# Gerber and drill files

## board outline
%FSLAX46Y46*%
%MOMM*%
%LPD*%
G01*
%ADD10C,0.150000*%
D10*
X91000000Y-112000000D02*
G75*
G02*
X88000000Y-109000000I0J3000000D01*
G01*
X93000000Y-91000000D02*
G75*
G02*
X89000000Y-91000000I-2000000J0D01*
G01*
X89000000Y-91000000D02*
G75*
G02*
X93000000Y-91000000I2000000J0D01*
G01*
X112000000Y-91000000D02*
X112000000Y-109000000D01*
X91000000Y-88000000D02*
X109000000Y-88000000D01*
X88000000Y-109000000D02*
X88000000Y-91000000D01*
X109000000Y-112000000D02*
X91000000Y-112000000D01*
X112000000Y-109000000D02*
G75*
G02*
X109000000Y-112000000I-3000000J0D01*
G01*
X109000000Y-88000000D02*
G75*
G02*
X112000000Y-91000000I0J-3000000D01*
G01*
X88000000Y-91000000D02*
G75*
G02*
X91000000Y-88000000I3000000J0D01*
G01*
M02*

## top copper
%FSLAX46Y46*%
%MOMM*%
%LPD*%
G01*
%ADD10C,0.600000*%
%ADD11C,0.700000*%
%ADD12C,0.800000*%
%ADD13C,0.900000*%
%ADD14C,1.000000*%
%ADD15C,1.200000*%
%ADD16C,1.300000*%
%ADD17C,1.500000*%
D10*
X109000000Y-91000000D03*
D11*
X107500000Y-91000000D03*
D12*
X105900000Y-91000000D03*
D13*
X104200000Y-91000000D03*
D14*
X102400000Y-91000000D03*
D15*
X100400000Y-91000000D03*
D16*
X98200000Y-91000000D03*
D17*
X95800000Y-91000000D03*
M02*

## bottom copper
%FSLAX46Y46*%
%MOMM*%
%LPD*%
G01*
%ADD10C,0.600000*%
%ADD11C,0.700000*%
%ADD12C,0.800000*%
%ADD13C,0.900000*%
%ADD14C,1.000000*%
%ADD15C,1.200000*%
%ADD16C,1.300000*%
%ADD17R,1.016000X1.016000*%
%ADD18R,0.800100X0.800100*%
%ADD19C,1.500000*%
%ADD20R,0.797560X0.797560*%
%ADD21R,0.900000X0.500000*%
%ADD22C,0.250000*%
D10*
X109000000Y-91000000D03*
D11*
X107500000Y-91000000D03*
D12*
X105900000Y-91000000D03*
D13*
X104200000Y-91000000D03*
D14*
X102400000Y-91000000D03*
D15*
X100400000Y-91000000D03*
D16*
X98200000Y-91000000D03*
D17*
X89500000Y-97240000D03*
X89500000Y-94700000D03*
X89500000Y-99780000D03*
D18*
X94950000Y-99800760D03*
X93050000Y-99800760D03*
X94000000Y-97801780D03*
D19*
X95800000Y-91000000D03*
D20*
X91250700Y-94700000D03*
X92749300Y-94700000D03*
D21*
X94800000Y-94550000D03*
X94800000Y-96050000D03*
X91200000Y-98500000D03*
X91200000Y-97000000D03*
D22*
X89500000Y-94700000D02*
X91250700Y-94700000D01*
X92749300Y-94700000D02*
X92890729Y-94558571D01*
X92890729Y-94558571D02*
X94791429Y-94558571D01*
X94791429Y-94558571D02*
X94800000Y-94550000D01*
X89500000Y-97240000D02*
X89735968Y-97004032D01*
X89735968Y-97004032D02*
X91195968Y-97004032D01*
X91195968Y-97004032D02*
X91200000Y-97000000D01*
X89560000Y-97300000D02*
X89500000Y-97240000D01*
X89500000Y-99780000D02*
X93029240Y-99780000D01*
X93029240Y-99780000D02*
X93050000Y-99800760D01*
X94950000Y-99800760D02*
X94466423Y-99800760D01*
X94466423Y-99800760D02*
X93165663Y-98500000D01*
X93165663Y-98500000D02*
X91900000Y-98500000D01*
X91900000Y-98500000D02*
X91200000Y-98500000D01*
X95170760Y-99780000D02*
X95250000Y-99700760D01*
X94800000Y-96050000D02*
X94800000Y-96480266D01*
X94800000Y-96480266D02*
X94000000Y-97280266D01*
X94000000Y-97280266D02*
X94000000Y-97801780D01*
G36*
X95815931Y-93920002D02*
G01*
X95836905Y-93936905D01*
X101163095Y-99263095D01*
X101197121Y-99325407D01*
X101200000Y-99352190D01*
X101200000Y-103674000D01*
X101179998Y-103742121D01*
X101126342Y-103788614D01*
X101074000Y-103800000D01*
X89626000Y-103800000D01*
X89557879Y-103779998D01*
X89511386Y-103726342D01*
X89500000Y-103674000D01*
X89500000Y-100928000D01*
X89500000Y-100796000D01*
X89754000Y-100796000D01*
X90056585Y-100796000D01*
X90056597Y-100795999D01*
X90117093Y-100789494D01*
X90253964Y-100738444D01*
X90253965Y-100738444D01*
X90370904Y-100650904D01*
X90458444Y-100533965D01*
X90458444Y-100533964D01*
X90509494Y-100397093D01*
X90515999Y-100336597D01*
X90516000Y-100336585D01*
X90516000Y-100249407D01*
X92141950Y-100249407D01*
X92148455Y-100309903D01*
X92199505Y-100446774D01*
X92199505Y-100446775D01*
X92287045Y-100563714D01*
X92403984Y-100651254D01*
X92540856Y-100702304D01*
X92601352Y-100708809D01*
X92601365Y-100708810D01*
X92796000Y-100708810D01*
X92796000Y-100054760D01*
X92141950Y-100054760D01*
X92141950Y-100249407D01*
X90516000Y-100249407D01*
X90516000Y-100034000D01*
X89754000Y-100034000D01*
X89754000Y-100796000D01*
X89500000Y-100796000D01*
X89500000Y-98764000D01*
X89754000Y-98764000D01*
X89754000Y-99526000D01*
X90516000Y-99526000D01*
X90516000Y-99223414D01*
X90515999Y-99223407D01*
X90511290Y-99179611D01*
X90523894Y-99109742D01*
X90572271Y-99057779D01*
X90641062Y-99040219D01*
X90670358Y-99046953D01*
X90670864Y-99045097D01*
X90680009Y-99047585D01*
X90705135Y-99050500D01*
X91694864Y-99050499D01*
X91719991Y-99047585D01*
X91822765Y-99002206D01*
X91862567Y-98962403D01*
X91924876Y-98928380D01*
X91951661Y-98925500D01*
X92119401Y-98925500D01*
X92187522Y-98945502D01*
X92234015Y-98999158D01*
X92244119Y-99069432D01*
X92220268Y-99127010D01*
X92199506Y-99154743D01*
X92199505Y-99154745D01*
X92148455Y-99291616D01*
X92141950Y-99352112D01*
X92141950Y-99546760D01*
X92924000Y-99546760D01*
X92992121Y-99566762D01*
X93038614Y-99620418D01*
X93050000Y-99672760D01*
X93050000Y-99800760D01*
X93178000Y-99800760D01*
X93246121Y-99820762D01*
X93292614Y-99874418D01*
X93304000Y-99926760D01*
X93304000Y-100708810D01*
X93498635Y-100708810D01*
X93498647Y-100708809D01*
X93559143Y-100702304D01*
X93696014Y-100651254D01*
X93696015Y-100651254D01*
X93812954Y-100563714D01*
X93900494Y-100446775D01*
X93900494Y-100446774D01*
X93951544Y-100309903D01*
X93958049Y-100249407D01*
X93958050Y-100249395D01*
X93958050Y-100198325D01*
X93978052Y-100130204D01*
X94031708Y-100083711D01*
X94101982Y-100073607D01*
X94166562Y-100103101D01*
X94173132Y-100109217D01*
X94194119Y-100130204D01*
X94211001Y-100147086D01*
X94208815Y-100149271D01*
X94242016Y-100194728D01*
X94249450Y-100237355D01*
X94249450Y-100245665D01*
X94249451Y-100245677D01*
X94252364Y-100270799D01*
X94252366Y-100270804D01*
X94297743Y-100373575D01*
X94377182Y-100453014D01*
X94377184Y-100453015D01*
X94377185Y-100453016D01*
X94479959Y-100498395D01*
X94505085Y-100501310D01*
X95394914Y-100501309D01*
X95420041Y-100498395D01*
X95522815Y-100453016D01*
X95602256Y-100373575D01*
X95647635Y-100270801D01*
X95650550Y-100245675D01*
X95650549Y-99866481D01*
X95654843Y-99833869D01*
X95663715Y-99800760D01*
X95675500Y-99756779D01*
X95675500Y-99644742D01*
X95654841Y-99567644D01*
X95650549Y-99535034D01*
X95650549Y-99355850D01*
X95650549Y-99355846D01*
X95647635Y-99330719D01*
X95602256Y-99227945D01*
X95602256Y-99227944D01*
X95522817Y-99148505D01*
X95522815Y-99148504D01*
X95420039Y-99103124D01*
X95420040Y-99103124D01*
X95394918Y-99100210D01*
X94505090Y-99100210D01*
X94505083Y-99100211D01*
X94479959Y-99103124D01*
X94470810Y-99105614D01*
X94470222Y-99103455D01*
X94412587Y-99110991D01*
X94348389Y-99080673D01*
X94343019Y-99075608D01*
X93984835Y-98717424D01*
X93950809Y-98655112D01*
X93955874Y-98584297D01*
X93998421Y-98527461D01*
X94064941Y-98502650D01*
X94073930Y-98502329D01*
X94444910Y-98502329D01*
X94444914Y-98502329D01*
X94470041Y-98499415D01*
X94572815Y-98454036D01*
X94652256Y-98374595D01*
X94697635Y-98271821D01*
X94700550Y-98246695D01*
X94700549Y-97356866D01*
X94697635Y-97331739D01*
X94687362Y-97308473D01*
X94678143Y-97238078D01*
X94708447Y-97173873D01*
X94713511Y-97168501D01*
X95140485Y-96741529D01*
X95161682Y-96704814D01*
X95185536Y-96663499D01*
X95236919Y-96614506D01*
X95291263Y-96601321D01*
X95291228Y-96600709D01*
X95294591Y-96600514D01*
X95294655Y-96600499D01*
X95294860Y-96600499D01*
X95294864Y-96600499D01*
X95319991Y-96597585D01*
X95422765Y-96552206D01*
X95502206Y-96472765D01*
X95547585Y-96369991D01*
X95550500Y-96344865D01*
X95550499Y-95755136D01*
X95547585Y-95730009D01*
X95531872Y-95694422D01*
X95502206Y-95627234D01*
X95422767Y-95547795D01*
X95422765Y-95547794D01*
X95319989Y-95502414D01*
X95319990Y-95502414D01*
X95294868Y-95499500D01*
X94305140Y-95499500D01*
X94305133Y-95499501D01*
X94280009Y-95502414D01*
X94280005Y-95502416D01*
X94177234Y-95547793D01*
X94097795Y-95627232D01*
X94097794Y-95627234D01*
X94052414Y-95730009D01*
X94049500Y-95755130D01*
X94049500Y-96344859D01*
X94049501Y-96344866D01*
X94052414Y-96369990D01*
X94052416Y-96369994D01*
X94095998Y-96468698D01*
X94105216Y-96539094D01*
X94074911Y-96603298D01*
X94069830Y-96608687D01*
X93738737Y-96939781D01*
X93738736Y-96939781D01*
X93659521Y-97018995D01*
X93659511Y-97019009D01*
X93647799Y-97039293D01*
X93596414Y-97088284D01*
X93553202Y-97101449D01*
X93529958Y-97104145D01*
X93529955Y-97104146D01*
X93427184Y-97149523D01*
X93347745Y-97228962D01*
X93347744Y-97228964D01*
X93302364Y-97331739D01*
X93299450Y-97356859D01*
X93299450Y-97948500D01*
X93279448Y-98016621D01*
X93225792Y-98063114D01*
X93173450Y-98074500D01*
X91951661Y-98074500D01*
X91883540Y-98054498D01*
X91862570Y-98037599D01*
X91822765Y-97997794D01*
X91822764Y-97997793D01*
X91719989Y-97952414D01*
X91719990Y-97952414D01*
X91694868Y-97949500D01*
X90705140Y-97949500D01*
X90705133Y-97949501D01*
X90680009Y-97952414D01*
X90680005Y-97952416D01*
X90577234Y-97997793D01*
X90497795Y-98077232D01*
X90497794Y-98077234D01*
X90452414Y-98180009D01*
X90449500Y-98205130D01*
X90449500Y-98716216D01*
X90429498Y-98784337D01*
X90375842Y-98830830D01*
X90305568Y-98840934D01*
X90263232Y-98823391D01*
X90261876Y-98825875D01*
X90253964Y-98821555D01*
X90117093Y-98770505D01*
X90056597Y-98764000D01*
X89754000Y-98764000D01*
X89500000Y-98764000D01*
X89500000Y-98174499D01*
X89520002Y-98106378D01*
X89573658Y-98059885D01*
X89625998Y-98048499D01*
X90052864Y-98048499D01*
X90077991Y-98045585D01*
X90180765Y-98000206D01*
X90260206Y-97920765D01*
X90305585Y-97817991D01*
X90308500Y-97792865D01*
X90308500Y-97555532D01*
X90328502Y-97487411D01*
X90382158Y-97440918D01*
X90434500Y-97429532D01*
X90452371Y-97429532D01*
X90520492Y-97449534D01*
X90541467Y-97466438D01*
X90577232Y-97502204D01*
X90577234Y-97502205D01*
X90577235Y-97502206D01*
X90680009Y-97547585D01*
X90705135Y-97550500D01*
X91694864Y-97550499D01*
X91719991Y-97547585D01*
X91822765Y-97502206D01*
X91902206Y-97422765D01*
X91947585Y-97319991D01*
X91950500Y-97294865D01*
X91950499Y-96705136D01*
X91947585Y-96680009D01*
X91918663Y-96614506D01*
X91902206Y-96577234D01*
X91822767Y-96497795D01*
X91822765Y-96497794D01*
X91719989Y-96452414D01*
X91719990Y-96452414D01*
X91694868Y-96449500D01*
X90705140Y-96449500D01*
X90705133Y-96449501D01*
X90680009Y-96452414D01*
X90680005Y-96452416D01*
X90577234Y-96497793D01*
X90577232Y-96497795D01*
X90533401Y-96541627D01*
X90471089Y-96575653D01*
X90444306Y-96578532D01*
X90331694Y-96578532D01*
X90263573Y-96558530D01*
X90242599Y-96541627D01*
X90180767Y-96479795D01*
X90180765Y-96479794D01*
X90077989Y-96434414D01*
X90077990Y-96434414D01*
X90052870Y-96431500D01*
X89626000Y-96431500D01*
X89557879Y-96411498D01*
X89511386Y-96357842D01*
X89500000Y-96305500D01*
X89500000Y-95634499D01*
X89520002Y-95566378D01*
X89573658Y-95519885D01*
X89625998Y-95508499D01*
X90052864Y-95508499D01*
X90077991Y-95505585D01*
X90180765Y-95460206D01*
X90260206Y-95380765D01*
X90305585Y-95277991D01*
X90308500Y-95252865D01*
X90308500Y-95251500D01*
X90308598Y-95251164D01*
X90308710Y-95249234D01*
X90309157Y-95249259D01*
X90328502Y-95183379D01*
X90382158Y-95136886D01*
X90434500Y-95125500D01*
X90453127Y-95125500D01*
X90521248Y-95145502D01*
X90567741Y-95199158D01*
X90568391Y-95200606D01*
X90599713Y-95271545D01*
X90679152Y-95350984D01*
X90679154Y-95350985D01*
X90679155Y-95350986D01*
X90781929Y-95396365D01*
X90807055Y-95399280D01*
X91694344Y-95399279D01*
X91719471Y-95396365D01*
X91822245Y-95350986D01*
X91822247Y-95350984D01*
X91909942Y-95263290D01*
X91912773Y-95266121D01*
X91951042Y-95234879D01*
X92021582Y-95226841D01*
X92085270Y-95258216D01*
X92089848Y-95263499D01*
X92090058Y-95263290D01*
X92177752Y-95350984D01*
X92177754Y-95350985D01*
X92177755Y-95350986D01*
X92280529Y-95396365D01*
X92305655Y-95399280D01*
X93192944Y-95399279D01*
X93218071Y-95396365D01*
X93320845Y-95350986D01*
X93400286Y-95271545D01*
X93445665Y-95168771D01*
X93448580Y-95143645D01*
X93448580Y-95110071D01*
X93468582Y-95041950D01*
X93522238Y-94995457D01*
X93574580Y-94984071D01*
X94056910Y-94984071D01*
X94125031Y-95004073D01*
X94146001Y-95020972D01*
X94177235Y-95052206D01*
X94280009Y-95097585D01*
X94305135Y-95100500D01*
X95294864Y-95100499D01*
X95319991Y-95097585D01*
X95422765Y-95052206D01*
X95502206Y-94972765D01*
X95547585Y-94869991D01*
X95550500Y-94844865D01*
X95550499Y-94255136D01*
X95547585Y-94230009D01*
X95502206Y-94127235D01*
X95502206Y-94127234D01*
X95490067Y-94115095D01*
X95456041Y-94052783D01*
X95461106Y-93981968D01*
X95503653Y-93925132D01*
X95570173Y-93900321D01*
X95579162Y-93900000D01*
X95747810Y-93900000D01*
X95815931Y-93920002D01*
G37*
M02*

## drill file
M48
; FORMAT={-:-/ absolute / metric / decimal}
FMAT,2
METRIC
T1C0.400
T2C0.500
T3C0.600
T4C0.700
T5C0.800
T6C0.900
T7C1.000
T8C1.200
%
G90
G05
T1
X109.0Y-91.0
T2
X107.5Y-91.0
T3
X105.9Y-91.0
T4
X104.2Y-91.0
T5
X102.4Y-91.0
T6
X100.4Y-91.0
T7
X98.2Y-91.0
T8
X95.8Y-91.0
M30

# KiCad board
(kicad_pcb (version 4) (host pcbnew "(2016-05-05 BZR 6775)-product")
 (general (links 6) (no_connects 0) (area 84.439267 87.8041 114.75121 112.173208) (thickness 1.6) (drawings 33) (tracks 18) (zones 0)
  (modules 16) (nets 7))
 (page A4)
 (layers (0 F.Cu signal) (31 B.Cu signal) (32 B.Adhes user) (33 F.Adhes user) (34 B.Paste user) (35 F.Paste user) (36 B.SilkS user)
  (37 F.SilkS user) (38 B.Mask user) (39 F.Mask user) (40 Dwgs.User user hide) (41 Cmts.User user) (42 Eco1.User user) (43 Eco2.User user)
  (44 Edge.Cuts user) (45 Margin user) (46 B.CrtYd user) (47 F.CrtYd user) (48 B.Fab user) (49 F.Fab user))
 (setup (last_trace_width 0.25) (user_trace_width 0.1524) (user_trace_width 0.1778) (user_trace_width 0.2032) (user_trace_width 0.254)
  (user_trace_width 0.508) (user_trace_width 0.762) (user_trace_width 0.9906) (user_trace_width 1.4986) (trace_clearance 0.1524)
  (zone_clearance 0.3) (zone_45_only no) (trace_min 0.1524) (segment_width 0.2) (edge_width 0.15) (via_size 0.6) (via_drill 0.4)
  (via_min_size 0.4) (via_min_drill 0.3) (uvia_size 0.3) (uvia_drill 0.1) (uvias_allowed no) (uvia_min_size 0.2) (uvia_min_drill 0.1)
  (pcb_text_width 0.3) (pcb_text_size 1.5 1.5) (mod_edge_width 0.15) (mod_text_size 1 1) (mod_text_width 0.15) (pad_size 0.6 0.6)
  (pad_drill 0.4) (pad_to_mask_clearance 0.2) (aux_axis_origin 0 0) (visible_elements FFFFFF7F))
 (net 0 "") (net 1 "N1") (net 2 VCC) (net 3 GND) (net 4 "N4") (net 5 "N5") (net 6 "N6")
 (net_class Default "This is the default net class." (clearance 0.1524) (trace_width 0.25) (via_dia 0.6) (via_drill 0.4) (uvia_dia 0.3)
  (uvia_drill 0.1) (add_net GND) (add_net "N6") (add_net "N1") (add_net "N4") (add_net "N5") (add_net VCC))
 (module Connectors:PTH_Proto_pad (layer F.Cu) (at 109 91)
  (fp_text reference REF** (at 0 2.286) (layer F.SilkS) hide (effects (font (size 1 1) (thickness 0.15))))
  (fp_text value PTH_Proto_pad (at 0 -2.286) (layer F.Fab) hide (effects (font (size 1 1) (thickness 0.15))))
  (pad 1 thru_hole circle (at 0 0) (size 0.6 0.6) (drill 0.4) (layers *.Cu *.Mask F.SilkS)))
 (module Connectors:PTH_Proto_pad (layer F.Cu) (at 107.5 91)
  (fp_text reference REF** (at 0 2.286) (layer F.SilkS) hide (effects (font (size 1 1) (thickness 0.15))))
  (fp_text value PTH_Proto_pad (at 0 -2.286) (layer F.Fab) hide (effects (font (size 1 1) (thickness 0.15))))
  (pad 1 thru_hole circle (at 0 0) (size 0.7 0.7) (drill 0.5) (layers *.Cu *.Mask F.SilkS)))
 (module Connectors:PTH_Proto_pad (layer F.Cu) (at 105.9 91)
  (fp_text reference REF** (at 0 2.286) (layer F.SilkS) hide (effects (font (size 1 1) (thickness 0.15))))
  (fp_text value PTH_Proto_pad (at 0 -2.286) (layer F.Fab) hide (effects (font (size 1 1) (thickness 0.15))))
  (pad 1 thru_hole circle (at 0 0) (size 0.8 0.8) (drill 0.6) (layers *.Cu *.Mask F.SilkS)))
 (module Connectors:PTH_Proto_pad (layer F.Cu) (at 104.2 91)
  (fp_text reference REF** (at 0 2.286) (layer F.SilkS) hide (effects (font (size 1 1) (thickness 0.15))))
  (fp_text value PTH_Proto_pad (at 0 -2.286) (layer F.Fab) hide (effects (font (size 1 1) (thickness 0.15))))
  (pad 1 thru_hole circle (at 0 0) (size 0.9 0.9) (drill 0.7) (layers *.Cu *.Mask F.SilkS)))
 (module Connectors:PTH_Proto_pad (layer F.Cu) (at 102.4 91)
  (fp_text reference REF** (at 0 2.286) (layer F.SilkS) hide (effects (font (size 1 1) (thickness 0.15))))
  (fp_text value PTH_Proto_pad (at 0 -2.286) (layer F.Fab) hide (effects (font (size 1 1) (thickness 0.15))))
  (pad 1 thru_hole circle (at 0 0) (size 1 1) (drill 0.8) (layers *.Cu *.Mask F.SilkS)))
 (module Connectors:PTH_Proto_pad (layer F.Cu) (at 100.4 91)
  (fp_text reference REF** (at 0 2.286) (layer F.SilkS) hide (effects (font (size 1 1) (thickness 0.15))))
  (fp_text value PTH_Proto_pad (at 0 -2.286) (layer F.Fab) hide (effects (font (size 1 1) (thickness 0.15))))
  (pad 1 thru_hole circle (at 0 0) (size 1.2 1.2) (drill 0.9) (layers *.Cu *.Mask F.SilkS)))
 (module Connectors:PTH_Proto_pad (layer F.Cu) (at 98.2 91)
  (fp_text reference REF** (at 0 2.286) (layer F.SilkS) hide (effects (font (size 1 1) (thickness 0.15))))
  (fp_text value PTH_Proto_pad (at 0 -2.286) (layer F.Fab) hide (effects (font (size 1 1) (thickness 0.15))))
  (pad 1 thru_hole circle (at 0 0) (size 1.3 1.3) (drill 1) (layers *.Cu *.Mask F.SilkS)))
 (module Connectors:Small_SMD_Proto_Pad (layer B.Cu) (at 89.5 97.24)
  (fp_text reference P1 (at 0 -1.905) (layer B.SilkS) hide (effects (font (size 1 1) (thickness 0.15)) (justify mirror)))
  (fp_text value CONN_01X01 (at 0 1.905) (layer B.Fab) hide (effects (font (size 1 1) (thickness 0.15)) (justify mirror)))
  (pad 1 smd rect (at 0 0) (size 1.016 1.016) (layers B.Cu B.Paste B.Mask) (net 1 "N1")))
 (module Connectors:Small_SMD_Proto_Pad (layer B.Cu) (at 89.5 94.7)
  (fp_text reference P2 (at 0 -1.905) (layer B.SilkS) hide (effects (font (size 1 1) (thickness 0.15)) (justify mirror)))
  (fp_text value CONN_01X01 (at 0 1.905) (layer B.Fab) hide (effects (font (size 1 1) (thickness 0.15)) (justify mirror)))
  (pad 1 smd rect (at 0 0) (size 1.016 1.016) (layers B.Cu B.Paste B.Mask) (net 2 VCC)))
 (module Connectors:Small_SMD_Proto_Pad (layer B.Cu) (at 89.5 99.78)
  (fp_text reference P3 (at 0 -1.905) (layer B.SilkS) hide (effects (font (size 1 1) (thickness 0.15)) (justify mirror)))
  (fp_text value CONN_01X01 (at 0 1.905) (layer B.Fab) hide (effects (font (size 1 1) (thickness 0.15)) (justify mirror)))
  (pad 1 smd rect (at 0 0) (size 1.016 1.016) (layers B.Cu B.Paste B.Mask) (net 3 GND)))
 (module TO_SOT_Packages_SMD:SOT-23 (layer B.Cu) (at 94 98.8 180)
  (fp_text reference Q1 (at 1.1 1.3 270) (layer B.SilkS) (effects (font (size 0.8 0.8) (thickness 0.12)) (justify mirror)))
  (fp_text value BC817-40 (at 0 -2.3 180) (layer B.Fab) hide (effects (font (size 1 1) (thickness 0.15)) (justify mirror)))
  (pad 1 smd rect (at -0.95 -1.00076 180) (size 0.8001 0.8001) (layers B.Cu B.Paste B.Mask) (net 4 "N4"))
  (pad 2 smd rect (at 0.95 -1.00076 180) (size 0.8001 0.8001) (layers B.Cu B.Paste B.Mask) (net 3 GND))
  (pad 3 smd rect (at 0 0.99822 180) (size 0.8001 0.8001) (layers B.Cu B.Paste B.Mask) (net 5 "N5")))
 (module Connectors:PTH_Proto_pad (layer F.Cu) (at 95.8 91)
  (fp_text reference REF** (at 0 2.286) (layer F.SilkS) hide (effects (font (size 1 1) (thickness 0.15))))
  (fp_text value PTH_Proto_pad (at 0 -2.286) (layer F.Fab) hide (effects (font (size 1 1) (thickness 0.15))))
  (pad 1 thru_hole circle (at 0 0) (size 1.5 1.5) (drill 1.2) (layers *.Cu *.Mask F.SilkS)))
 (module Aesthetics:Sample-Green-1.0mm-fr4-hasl (layer B.Cu) (at 100 102.6 180)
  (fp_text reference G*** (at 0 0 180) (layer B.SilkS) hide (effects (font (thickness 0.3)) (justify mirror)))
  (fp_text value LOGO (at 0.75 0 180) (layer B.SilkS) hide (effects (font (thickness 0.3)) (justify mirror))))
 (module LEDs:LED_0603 (layer B.Cu) (at 92 94.7 180)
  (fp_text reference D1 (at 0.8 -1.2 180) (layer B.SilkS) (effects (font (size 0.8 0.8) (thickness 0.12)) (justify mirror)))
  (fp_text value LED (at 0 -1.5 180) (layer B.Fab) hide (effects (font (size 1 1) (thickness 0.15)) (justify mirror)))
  (pad 2 smd rect (at 0.7493 0) (size 0.79756 0.79756) (layers B.Cu B.Paste B.Mask) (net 2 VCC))
  (pad 1 smd rect (at -0.7493 0) (size 0.79756 0.79756) (layers B.Cu B.Paste B.Mask) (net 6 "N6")))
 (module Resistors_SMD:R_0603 (layer B.Cu) (at 94.8 95.3 270)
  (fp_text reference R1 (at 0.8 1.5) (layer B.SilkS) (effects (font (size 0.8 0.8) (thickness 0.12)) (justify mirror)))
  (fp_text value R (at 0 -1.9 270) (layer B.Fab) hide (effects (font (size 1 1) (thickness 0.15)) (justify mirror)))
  (pad 1 smd rect (at -0.75 0 270) (size 0.5 0.9) (layers B.Cu B.Paste B.Mask) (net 6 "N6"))
  (pad 2 smd rect (at 0.75 0 270) (size 0.5 0.9) (layers B.Cu B.Paste B.Mask) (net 5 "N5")))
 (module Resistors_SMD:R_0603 (layer B.Cu) (at 91.2 97.75 90)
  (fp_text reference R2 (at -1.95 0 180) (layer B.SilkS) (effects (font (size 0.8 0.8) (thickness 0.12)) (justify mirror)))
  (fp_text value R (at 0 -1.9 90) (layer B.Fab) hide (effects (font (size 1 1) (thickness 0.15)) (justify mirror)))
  (pad 1 smd rect (at -0.75 0 90) (size 0.5 0.9) (layers B.Cu B.Paste B.Mask) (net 4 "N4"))
  (pad 2 smd rect (at 0.75 0 90) (size 0.5 0.9) (layers B.Cu B.Paste B.Mask) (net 1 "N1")))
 (gr_arc (start 91 109) (end 91 112) (angle 90) (layer Edge.Cuts) (width 0.15))
 (gr_circle (center 91 91) (end 93 91) (layer Edge.Cuts) (width 0.15))
 (gr_line (start 112 91) (end 112 109) (layer Edge.Cuts) (width 0.15))
 (gr_line (start 91 88) (end 109 88) (layer Edge.Cuts) (width 0.15))
 (gr_line (start 88 109) (end 88 91) (layer Edge.Cuts) (width 0.15))
 (gr_line (start 109 112) (end 91 112) (layer Edge.Cuts) (width 0.15))
 (gr_arc (start 109 109) (end 112 109) (angle 90) (layer Edge.Cuts) (width 0.15))
 (gr_arc (start 109 91) (end 109 88) (angle 90) (layer Edge.Cuts) (width 0.15))
 (gr_arc (start 91 91) (end 88 91) (angle 90) (layer Edge.Cuts) (width 0.15))
 (segment (start 89.5 94.7) (end 91.2507 94.7) (width 0.25) (layer B.Cu) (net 2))
 (segment (start 92.7493 94.7) (end 92.890729 94.558571) (width 0.25) (layer B.Cu) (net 6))
 (segment (start 92.890729 94.558571) (end 94.791429 94.558571) (width 0.25) (layer B.Cu) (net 6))
 (segment (start 94.791429 94.558571) (end 94.8 94.55) (width 0.25) (layer B.Cu) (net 6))
 (segment (start 89.5 97.24) (end 89.735968 97.004032) (width 0.25) (layer B.Cu) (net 1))
 (segment (start 89.735968 97.004032) (end 91.195968 97.004032) (width 0.25) (layer B.Cu) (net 1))
 (segment (start 91.195968 97.004032) (end 91.2 97) (width 0.25) (layer B.Cu) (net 1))
 (segment (start 89.56 97.3) (end 89.5 97.24) (width 0.25) (layer B.Cu) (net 1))
 (segment (start 89.5 99.78) (end 93.02924 99.78) (width 0.25) (layer B.Cu) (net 3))
 (segment (start 93.02924 99.78) (end 93.05 99.80076) (width 0.25) (layer B.Cu) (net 3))
 (segment (start 94.95 99.80076) (end 94.466423 99.80076) (width 0.25) (layer B.Cu) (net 4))
 (segment (start 94.466423 99.80076) (end 93.165663 98.5) (width 0.25) (layer B.Cu) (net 4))
 (segment (start 93.165663 98.5) (end 91.9 98.5) (width 0.25) (layer B.Cu) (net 4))
 (segment (start 91.9 98.5) (end 91.2 98.5) (width 0.25) (layer B.Cu) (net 4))
 (segment (start 95.17076 99.78) (end 95.25 99.70076) (width 0.25) (layer B.Cu) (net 4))
 (segment (start 94.8 96.05) (end 94.8 96.480266) (width 0.25) (layer B.Cu) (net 5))
 (segment (start 94.8 96.480266) (end 94 97.280266) (width 0.25) (layer B.Cu) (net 5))
 (segment (start 94 97.280266) (end 94 97.80178) (width 0.25) (layer B.Cu) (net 5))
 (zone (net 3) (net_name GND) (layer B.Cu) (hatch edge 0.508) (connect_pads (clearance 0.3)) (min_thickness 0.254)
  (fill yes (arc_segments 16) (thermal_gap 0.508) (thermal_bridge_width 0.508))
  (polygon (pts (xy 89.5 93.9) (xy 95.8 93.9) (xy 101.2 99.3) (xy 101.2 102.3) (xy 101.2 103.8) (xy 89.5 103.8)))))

